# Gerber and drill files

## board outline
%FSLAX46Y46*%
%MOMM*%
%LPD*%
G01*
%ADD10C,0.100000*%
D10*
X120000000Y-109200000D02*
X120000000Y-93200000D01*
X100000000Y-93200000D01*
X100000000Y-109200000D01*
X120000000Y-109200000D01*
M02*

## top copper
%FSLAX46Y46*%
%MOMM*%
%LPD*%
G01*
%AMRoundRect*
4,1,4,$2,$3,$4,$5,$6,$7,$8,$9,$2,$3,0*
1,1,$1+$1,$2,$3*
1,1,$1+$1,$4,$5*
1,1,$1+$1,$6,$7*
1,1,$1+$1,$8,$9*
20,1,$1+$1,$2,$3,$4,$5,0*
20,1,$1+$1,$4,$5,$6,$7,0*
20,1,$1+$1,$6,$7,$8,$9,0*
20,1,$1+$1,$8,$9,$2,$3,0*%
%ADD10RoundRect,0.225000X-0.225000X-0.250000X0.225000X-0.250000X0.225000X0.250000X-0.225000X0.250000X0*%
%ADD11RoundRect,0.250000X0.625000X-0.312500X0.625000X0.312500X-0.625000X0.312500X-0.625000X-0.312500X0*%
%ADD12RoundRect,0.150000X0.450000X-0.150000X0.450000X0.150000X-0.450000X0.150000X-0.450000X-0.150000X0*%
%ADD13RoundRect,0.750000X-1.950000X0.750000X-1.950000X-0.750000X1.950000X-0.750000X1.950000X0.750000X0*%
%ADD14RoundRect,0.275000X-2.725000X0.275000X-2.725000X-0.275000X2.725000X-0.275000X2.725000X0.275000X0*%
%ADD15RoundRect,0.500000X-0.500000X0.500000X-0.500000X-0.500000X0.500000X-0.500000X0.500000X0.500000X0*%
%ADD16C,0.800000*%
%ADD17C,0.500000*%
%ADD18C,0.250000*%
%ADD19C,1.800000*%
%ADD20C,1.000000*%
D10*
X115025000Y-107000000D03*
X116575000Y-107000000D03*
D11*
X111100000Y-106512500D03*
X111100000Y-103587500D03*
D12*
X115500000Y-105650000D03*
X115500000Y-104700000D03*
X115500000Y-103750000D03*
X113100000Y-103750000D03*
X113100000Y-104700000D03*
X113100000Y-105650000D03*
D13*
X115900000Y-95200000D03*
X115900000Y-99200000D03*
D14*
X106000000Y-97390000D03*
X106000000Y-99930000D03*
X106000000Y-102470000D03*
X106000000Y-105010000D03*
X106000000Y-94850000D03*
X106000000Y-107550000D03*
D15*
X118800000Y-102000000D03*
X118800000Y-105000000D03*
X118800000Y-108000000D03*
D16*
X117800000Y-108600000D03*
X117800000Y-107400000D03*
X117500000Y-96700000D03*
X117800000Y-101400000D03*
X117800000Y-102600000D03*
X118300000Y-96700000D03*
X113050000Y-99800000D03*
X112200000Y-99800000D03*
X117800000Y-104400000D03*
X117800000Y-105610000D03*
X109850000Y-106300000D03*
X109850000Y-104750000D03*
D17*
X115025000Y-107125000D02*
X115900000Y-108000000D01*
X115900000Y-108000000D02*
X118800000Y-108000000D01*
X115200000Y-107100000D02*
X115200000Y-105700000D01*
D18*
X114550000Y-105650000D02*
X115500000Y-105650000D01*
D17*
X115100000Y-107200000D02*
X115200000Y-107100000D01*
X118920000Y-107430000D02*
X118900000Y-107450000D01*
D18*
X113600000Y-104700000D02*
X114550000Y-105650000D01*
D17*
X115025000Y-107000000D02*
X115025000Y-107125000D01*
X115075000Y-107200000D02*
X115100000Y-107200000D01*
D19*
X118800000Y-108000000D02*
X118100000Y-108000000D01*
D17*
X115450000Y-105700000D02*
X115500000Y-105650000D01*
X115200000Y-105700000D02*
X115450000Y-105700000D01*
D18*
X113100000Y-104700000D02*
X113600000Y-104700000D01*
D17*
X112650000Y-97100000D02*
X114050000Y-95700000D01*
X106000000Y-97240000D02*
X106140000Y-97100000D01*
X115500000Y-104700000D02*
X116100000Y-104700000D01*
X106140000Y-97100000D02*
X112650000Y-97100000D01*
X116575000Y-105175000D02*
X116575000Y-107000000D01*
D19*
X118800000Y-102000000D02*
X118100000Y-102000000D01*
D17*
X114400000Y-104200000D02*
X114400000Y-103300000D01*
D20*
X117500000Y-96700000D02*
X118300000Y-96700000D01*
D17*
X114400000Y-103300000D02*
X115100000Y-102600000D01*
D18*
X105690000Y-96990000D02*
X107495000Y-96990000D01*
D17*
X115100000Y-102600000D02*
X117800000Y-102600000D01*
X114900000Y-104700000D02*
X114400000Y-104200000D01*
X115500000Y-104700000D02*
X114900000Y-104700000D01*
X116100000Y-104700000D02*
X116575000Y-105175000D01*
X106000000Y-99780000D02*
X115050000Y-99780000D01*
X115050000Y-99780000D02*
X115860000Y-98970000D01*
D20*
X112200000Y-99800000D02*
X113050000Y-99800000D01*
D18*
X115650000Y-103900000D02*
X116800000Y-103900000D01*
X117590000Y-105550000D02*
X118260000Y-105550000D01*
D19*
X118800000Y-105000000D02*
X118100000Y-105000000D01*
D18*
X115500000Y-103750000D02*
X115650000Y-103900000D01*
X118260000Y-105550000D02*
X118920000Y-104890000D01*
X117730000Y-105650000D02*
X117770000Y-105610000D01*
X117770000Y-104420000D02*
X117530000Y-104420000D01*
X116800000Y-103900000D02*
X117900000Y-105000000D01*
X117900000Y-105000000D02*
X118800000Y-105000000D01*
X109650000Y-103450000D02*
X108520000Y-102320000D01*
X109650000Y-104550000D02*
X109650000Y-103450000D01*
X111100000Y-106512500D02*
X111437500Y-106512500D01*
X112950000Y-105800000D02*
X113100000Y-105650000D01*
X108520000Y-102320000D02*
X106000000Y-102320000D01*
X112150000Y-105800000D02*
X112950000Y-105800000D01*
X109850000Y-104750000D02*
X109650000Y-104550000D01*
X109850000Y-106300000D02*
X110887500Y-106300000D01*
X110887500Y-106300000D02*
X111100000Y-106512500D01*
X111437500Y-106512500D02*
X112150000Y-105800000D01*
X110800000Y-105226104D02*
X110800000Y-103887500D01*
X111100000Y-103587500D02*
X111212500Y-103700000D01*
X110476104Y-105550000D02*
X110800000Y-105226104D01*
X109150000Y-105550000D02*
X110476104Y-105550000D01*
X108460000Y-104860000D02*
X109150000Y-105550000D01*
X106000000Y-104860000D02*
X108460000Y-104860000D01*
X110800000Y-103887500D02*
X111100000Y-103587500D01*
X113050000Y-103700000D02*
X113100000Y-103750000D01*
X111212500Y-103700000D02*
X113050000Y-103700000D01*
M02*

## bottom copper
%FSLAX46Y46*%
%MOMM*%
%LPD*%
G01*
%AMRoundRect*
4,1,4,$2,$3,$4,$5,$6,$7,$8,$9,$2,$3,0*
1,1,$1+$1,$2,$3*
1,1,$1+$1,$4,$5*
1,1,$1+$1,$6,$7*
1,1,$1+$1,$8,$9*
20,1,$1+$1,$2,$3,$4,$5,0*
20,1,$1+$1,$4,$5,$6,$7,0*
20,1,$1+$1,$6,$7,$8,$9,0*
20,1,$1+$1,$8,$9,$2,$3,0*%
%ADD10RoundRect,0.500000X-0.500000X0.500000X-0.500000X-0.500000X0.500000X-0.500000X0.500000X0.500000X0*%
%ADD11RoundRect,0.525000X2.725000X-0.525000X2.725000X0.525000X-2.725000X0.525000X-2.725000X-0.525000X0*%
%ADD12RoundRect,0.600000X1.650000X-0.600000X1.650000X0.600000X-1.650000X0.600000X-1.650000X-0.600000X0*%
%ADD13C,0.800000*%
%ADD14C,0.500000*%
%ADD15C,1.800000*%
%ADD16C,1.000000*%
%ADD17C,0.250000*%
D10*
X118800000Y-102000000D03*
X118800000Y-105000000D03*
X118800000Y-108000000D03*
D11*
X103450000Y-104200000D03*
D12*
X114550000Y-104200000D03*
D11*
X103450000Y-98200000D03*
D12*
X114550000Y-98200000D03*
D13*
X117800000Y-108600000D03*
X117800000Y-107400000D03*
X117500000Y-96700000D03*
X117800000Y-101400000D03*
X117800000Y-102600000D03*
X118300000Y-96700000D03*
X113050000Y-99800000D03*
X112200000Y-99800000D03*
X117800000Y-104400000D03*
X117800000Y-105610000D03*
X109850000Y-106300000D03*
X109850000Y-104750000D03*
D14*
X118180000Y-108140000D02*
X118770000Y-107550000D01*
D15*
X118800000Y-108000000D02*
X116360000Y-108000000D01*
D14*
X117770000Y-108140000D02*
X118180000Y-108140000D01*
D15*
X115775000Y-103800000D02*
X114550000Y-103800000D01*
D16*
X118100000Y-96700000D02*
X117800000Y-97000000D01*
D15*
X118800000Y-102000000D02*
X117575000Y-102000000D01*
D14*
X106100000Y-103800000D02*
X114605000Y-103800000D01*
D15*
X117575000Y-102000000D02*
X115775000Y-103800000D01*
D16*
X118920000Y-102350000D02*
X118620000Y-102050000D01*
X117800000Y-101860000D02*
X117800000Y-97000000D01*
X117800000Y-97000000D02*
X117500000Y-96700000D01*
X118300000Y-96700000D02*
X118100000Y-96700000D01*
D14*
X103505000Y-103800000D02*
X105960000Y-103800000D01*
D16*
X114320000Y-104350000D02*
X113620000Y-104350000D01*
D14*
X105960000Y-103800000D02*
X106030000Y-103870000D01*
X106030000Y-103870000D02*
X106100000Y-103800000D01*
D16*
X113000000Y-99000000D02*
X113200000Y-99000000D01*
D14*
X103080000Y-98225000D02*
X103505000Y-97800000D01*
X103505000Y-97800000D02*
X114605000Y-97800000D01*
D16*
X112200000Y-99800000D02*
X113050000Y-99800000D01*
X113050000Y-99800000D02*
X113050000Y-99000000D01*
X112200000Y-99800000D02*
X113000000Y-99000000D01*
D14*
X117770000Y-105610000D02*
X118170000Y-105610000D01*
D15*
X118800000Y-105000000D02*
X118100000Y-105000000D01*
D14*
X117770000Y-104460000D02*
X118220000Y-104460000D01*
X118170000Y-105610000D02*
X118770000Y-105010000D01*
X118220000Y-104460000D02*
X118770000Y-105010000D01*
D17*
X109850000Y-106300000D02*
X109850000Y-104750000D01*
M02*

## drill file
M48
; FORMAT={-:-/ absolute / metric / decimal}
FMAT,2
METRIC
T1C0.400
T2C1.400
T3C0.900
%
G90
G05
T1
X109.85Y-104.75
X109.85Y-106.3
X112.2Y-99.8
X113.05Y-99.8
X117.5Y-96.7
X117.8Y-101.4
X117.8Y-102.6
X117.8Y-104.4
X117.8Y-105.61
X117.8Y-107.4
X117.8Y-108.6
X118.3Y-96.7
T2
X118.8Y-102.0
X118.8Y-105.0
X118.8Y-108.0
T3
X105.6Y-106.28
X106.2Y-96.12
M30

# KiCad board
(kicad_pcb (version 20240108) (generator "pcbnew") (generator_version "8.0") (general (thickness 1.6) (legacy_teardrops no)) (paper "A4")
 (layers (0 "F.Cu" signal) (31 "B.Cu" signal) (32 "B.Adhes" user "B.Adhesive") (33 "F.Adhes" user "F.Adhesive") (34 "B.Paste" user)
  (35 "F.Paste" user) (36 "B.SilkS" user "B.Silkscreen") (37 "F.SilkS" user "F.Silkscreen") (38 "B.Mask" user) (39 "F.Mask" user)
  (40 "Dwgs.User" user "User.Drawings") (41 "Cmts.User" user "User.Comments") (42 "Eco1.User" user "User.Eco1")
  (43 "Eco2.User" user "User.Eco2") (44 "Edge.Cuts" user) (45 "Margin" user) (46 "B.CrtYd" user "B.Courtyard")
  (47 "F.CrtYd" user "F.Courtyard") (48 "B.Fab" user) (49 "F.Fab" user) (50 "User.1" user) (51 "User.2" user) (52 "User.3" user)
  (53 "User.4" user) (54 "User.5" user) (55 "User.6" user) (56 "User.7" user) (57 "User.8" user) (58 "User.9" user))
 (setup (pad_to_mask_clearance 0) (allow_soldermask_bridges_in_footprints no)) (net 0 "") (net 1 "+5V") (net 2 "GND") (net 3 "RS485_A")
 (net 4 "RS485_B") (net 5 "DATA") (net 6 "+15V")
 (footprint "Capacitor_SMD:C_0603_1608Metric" (layer "F.Cu") (at 115.8 107)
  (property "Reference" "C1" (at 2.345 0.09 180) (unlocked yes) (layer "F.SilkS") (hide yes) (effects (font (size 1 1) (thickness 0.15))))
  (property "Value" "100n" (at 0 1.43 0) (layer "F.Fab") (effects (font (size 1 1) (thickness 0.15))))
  (pad "1" smd roundrect (at -0.775 0) (size 0.9 0.95) (layers "F.Cu" "F.Paste" "F.Mask") (roundrect_rratio 0.25) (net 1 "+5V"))
  (pad "2" smd roundrect (at 0.775 0) (size 0.9 0.95) (layers "F.Cu" "F.Paste" "F.Mask") (roundrect_rratio 0.25) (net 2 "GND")))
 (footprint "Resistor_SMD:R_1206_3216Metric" (layer "F.Cu") (at 111.1 105.05 90)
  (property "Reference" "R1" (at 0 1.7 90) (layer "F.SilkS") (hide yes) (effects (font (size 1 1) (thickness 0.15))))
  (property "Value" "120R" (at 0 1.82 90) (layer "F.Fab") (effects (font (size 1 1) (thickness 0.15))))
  (pad "1" smd roundrect (at -1.4625 0 90) (size 1.125 1.75) (layers "F.Cu" "F.Paste" "F.Mask") (roundrect_rratio 0.222222)
   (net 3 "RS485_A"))
  (pad "2" smd roundrect (at 1.4625 0 90) (size 1.125 1.75) (layers "F.Cu" "F.Paste" "F.Mask") (roundrect_rratio 0.222222) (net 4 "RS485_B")))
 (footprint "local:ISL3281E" (layer "F.Cu") (at 114.3 104.7 90)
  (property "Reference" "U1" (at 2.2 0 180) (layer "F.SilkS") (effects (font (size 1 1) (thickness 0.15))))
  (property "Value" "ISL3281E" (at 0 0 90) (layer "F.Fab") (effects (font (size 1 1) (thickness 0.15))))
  (pad "1" smd roundrect (at -0.95 1.2 90) (size 0.6 1.2) (layers "F.Cu" "F.Paste" "F.Mask") (roundrect_rratio 0.25) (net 1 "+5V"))
  (pad "2" smd roundrect (at 0 1.2 90) (size 0.6 1.2) (layers "F.Cu" "F.Paste" "F.Mask") (roundrect_rratio 0.25) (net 2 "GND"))
  (pad "3" smd roundrect (at 0.95 1.2 90) (size 0.6 1.2) (layers "F.Cu" "F.Paste" "F.Mask") (roundrect_rratio 0.25) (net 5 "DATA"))
  (pad "4" smd roundrect (at 0.95 -1.2 90) (size 0.6 1.2) (layers "F.Cu" "F.Paste" "F.Mask") (roundrect_rratio 0.25) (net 4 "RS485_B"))
  (pad "5" smd roundrect (at 0 -1.2 90) (size 0.6 1.2) (layers "F.Cu" "F.Paste" "F.Mask") (roundrect_rratio 0.25) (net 1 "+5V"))
  (pad "6" smd roundrect (at -0.95 -1.2 90) (size 0.6 1.2) (layers "F.Cu" "F.Paste" "F.Mask") (roundrect_rratio 0.25) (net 3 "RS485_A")))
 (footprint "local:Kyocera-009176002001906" (layer "F.Cu") (at 115.9 97.2 -90)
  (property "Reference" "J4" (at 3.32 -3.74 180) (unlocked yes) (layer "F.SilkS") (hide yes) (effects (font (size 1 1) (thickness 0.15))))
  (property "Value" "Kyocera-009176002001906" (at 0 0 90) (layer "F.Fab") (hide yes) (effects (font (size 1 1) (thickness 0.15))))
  (pad "1" smd roundrect (at -2 0 270) (size 3 5.4) (layers "F.Cu" "F.Paste" "F.Mask") (roundrect_rratio 0.25) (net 2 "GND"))
  (pad "2" smd roundrect (at 2 0 270) (size 3 5.4) (layers "F.Cu" "F.Paste" "F.Mask") (roundrect_rratio 0.25) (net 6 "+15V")))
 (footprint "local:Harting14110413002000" (layer "F.Cu") (at 106 101.2 -90)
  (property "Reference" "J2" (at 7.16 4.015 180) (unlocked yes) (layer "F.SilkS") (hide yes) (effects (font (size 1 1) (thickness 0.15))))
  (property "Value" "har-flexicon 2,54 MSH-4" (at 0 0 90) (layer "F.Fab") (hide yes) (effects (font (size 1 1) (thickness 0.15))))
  (pad "" np_thru_hole circle (at -5.08 -0.2 270) (size 0.9 0.9) (drill 0.9) (layers "*.Cu" "*.Mask"))
  (pad "" np_thru_hole circle (at 5.08 0.4 270) (size 0.9 0.9) (drill 0.9) (layers "*.Cu" "*.Mask"))
  (pad "1" smd roundrect (at -3.81 0 270) (size 1.1 6) (layers "F.Cu" "F.Paste" "F.Mask") (roundrect_rratio 0.25) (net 2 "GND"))
  (pad "2" smd roundrect (at -1.27 0 270) (size 1.1 6) (layers "F.Cu" "F.Paste" "F.Mask") (roundrect_rratio 0.25) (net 6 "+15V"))
  (pad "3" smd roundrect (at 1.27 0 270) (size 1.1 6) (layers "F.Cu" "F.Paste" "F.Mask") (roundrect_rratio 0.25) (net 3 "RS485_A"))
  (pad "4" smd roundrect (at 3.81 0 270) (size 1.1 6) (layers "F.Cu" "F.Paste" "F.Mask") (roundrect_rratio 0.25) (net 4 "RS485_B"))
  (pad "MP1" smd roundrect (at -6.35 0 270) (size 1.1 6) (layers "F.Cu" "F.Paste" "F.Mask") (roundrect_rratio 0.25))
  (pad "MP2" smd roundrect (at 6.35 0 270) (size 1.1 6) (layers "F.Cu" "F.Paste" "F.Mask") (roundrect_rratio 0.25)))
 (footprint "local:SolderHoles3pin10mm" (layer "F.Cu") (at 118.8 105 -90)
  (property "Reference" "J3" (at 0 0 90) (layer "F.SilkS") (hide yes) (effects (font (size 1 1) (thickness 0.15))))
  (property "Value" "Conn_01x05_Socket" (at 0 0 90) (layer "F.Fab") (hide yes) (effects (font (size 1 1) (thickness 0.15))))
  (pad "1" thru_hole roundrect (at -3 0 270) (size 2 2) (drill 1.4) (layers "*.Cu" "*.Mask") (remove_unused_layers yes)
   (keep_end_layers yes) (zone_layer_connections) (roundrect_rratio 0.25) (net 2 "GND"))
  (pad "2" thru_hole roundrect (at 0 0 270) (size 2 2) (drill 1.4) (layers "*.Cu" "*.Mask") (remove_unused_layers yes) (keep_end_layers yes)
   (zone_layer_connections) (roundrect_rratio 0.25) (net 5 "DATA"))
  (pad "3" thru_hole roundrect (at 3 0 270) (size 2 2) (drill 1.4) (layers "*.Cu" "*.Mask") (remove_unused_layers yes) (keep_end_layers yes)
   (zone_layer_connections) (roundrect_rratio 0.25) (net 1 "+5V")))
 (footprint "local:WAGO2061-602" (layer "B.Cu") (at 108.2 101.2 90)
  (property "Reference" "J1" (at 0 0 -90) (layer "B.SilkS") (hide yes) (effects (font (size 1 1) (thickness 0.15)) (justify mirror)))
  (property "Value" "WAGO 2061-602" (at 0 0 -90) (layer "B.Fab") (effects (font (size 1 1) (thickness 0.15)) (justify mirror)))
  (pad "1" smd roundrect (at -3 -4.75 90) (size 2.1 6.5) (layers "B.Cu" "B.Paste" "B.Mask") (roundrect_rratio 0.25) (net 2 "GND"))
  (pad "1" smd roundrect (at -3 6.35 90) (size 2.4 4.5) (layers "B.Cu" "B.Paste" "B.Mask") (roundrect_rratio 0.25) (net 2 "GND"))
  (pad "2" smd roundrect (at 3 -4.75 90) (size 2.1 6.5) (layers "B.Cu" "B.Paste" "B.Mask") (roundrect_rratio 0.25) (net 6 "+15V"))
  (pad "2" smd roundrect (at 3 6.35 90) (size 2.4 4.5) (layers "B.Cu" "B.Paste" "B.Mask") (roundrect_rratio 0.25) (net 6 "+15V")))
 (gr_poly (pts (xy 120 109.2) (xy 120 93.2) (xy 100 93.2) (xy 100 109.2)) (stroke (width 0.1) (type solid)) (fill none) (layer "Edge.Cuts"))
 (segment (start 115.025 107.125) (end 115.9 108) (width 0.5) (layer "F.Cu") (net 1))
 (segment (start 115.9 108) (end 118.8 108) (width 0.5) (layer "F.Cu") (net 1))
 (segment (start 115.2 107.1) (end 115.2 105.7) (width 0.5) (layer "F.Cu") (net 1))
 (segment (start 114.55 105.65) (end 115.5 105.65) (width 0.25) (layer "F.Cu") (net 1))
 (segment (start 115.1 107.2) (end 115.2 107.1) (width 0.5) (layer "F.Cu") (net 1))
 (segment (start 118.92 107.43) (end 118.9 107.45) (width 0.5) (layer "F.Cu") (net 1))
 (segment (start 113.6 104.7) (end 114.55 105.65) (width 0.25) (layer "F.Cu") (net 1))
 (segment (start 115.025 107) (end 115.025 107.125) (width 0.5) (layer "F.Cu") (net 1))
 (segment (start 115.075 107.2) (end 115.1 107.2) (width 0.5) (layer "F.Cu") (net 1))
 (segment (start 118.8 108) (end 118.1 108) (width 1.8) (layer "F.Cu") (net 1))
 (segment (start 115.45 105.7) (end 115.5 105.65) (width 0.5) (layer "F.Cu") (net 1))
 (segment (start 115.2 105.7) (end 115.45 105.7) (width 0.5) (layer "F.Cu") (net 1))
 (segment (start 113.1 104.7) (end 113.6 104.7) (width 0.25) (layer "F.Cu") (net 1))
 (via (at 117.8 108.6) (size 0.8) (drill 0.4) (layers "F.Cu" "B.Cu") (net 1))
 (via (at 117.8 107.4) (size 0.8) (drill 0.4) (layers "F.Cu" "B.Cu") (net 1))
 (segment (start 118.18 108.14) (end 118.77 107.55) (width 0.5) (layer "B.Cu") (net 1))
 (segment (start 118.8 108) (end 116.36 108) (width 1.8) (layer "B.Cu") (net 1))
 (segment (start 117.77 108.14) (end 118.18 108.14) (width 0.5) (layer "B.Cu") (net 1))
 (segment (start 112.65 97.1) (end 114.05 95.7) (width 0.5) (layer "F.Cu") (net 2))
 (segment (start 106 97.24) (end 106.14 97.1) (width 0.5) (layer "F.Cu") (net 2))
 (segment (start 115.5 104.7) (end 116.1 104.7) (width 0.5) (layer "F.Cu") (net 2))
 (segment (start 106.14 97.1) (end 112.65 97.1) (width 0.5) (layer "F.Cu") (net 2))
 (segment (start 116.575 105.175) (end 116.575 107) (width 0.5) (layer "F.Cu") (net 2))
 (segment (start 118.8 102) (end 118.1 102) (width 1.8) (layer "F.Cu") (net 2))
 (segment (start 114.4 104.2) (end 114.4 103.3) (width 0.5) (layer "F.Cu") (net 2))
 (segment (start 117.5 96.7) (end 118.3 96.7) (width 1) (layer "F.Cu") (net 2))
 (segment (start 114.4 103.3) (end 115.1 102.6) (width 0.5) (layer "F.Cu") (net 2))
 (segment (start 105.69 96.99) (end 107.495 96.99) (width 0.25) (layer "F.Cu") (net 2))
 (segment (start 115.1 102.6) (end 117.8 102.6) (width 0.5) (layer "F.Cu") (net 2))
 (segment (start 114.9 104.7) (end 114.4 104.2) (width 0.5) (layer "F.Cu") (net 2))
 (segment (start 115.5 104.7) (end 114.9 104.7) (width 0.5) (layer "F.Cu") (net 2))
 (segment (start 116.1 104.7) (end 116.575 105.175) (width 0.5) (layer "F.Cu") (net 2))
 (via (at 117.5 96.7) (size 0.8) (drill 0.4) (layers "F.Cu" "B.Cu") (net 2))
 (via (at 117.8 101.4) (size 0.8) (drill 0.4) (layers "F.Cu" "B.Cu") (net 2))
 (via (at 117.8 102.6) (size 0.8) (drill 0.4) (layers "F.Cu" "B.Cu") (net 2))
 (via (at 118.3 96.7) (size 0.8) (drill 0.4) (layers "F.Cu" "B.Cu") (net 2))
 (segment (start 115.775 103.8) (end 114.55 103.8) (width 1.8) (layer "B.Cu") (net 2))
 (segment (start 118.1 96.7) (end 117.8 97) (width 1) (layer "B.Cu") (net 2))
 (segment (start 118.8 102) (end 117.575 102) (width 1.8) (layer "B.Cu") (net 2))
 (segment (start 106.1 103.8) (end 114.605 103.8) (width 0.5) (layer "B.Cu") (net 2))
 (segment (start 117.575 102) (end 115.775 103.8) (width 1.8) (layer "B.Cu") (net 2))
 (segment (start 118.92 102.35) (end 118.62 102.05) (width 1) (layer "B.Cu") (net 2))
 (segment (start 117.8 101.86) (end 117.8 97) (width 1) (layer "B.Cu") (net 2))
 (segment (start 117.8 97) (end 117.5 96.7) (width 1) (layer "B.Cu") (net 2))
 (segment (start 118.3 96.7) (end 118.1 96.7) (width 1) (layer "B.Cu") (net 2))
 (segment (start 103.505 103.8) (end 105.96 103.8) (width 0.5) (layer "B.Cu") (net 2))
 (segment (start 114.32 104.35) (end 113.62 104.35) (width 1) (layer "B.Cu") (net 2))
 (segment (start 105.96 103.8) (end 106.03 103.87) (width 0.5) (layer "B.Cu") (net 2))
 (segment (start 106.03 103.87) (end 106.1 103.8) (width 0.5) (layer "B.Cu") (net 2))
 (segment (start 106 99.78) (end 115.05 99.78) (width 0.5) (layer "F.Cu") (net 6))
 (segment (start 115.05 99.78) (end 115.86 98.97) (width 0.5) (layer "F.Cu") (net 6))
 (segment (start 112.2 99.8) (end 113.05 99.8) (width 1) (layer "F.Cu") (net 6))
 (via (at 113.05 99.8) (size 0.8) (drill 0.4) (layers "F.Cu" "B.Cu") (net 6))
 (via (at 112.2 99.8) (size 0.8) (drill 0.4) (layers "F.Cu" "B.Cu") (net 6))
 (segment (start 113 99) (end 113.2 99) (width 1) (layer "B.Cu") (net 6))
 (segment (start 103.08 98.225) (end 103.505 97.8) (width 0.5) (layer "B.Cu") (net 6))
 (segment (start 103.505 97.8) (end 114.605 97.8) (width 0.5) (layer "B.Cu") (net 6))
 (segment (start 112.2 99.8) (end 113.05 99.8) (width 1) (layer "B.Cu") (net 6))
 (segment (start 113.05 99.8) (end 113.05 99) (width 1) (layer "B.Cu") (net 6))
 (segment (start 112.2 99.8) (end 113 99) (width 1) (layer "B.Cu") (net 6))
 (segment (start 115.65 103.9) (end 116.8 103.9) (width 0.25) (layer "F.Cu") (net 5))
 (segment (start 117.59 105.55) (end 118.26 105.55) (width 0.25) (layer "F.Cu") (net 5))
 (segment (start 118.8 105) (end 118.1 105) (width 1.8) (layer "F.Cu") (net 5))
 (segment (start 115.5 103.75) (end 115.65 103.9) (width 0.25) (layer "F.Cu") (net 5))
 (segment (start 118.26 105.55) (end 118.92 104.89) (width 0.25) (layer "F.Cu") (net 5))
 (segment (start 117.73 105.65) (end 117.77 105.61) (width 0.25) (layer "F.Cu") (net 5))
 (segment (start 117.77 104.42) (end 117.53 104.42) (width 0.25) (layer "F.Cu") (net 5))
 (segment (start 116.8 103.9) (end 117.9 105) (width 0.25) (layer "F.Cu") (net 5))
 (segment (start 117.9 105) (end 118.8 105) (width 0.25) (layer "F.Cu") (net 5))
 (via (at 117.8 104.4) (size 0.8) (drill 0.4) (layers "F.Cu" "B.Cu") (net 5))
 (via (at 117.8 105.61) (size 0.8) (drill 0.4) (layers "F.Cu" "B.Cu") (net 5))
 (segment (start 117.77 105.61) (end 118.17 105.61) (width 0.5) (layer "B.Cu") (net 5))
 (segment (start 118.8 105) (end 118.1 105) (width 1.8) (layer "B.Cu") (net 5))
 (segment (start 117.77 104.46) (end 118.22 104.46) (width 0.5) (layer "B.Cu") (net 5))
 (segment (start 118.17 105.61) (end 118.77 105.01) (width 0.5) (layer "B.Cu") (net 5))
 (segment (start 118.22 104.46) (end 118.77 105.01) (width 0.5) (layer "B.Cu") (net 5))
 (segment (start 109.65 103.45) (end 108.52 102.32) (width 0.25) (layer "F.Cu") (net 3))
 (segment (start 109.65 104.55) (end 109.65 103.45) (width 0.25) (layer "F.Cu") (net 3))
 (segment (start 111.1 106.5125) (end 111.4375 106.5125) (width 0.25) (layer "F.Cu") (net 3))
 (segment (start 112.95 105.8) (end 113.1 105.65) (width 0.25) (layer "F.Cu") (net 3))
 (segment (start 108.52 102.32) (end 106 102.32) (width 0.25) (layer "F.Cu") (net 3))
 (segment (start 112.15 105.8) (end 112.95 105.8) (width 0.25) (layer "F.Cu") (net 3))
 (segment (start 109.85 104.75) (end 109.65 104.55) (width 0.25) (layer "F.Cu") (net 3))
 (segment (start 109.85 106.3) (end 110.8875 106.3) (width 0.25) (layer "F.Cu") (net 3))
 (segment (start 110.8875 106.3) (end 111.1 106.5125) (width 0.25) (layer "F.Cu") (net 3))
 (segment (start 111.4375 106.5125) (end 112.15 105.8) (width 0.25) (layer "F.Cu") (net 3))
 (via (at 109.85 106.3) (size 0.8) (drill 0.4) (layers "F.Cu" "B.Cu") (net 3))
 (via (at 109.85 104.75) (size 0.8) (drill 0.4) (layers "F.Cu" "B.Cu") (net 3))
 (segment (start 109.85 106.3) (end 109.85 104.75) (width 0.25) (layer "B.Cu") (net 3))
 (segment (start 110.8 105.226104) (end 110.8 103.8875) (width 0.25) (layer "F.Cu") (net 4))
 (segment (start 111.1 103.5875) (end 111.2125 103.7) (width 0.25) (layer "F.Cu") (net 4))
 (segment (start 110.476104 105.55) (end 110.8 105.226104) (width 0.25) (layer "F.Cu") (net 4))
 (segment (start 109.15 105.55) (end 110.476104 105.55) (width 0.25) (layer "F.Cu") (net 4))
 (segment (start 108.46 104.86) (end 109.15 105.55) (width 0.25) (layer "F.Cu") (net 4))
 (segment (start 106 104.86) (end 108.46 104.86) (width 0.25) (layer "F.Cu") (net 4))
 (segment (start 110.8 103.8875) (end 111.1 103.5875) (width 0.25) (layer "F.Cu") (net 4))
 (segment (start 113.05 103.7) (end 113.1 103.75) (width 0.25) (layer "F.Cu") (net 4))
 (segment (start 111.2125 103.7) (end 113.05 103.7) (width 0.25) (layer "F.Cu") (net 4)))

